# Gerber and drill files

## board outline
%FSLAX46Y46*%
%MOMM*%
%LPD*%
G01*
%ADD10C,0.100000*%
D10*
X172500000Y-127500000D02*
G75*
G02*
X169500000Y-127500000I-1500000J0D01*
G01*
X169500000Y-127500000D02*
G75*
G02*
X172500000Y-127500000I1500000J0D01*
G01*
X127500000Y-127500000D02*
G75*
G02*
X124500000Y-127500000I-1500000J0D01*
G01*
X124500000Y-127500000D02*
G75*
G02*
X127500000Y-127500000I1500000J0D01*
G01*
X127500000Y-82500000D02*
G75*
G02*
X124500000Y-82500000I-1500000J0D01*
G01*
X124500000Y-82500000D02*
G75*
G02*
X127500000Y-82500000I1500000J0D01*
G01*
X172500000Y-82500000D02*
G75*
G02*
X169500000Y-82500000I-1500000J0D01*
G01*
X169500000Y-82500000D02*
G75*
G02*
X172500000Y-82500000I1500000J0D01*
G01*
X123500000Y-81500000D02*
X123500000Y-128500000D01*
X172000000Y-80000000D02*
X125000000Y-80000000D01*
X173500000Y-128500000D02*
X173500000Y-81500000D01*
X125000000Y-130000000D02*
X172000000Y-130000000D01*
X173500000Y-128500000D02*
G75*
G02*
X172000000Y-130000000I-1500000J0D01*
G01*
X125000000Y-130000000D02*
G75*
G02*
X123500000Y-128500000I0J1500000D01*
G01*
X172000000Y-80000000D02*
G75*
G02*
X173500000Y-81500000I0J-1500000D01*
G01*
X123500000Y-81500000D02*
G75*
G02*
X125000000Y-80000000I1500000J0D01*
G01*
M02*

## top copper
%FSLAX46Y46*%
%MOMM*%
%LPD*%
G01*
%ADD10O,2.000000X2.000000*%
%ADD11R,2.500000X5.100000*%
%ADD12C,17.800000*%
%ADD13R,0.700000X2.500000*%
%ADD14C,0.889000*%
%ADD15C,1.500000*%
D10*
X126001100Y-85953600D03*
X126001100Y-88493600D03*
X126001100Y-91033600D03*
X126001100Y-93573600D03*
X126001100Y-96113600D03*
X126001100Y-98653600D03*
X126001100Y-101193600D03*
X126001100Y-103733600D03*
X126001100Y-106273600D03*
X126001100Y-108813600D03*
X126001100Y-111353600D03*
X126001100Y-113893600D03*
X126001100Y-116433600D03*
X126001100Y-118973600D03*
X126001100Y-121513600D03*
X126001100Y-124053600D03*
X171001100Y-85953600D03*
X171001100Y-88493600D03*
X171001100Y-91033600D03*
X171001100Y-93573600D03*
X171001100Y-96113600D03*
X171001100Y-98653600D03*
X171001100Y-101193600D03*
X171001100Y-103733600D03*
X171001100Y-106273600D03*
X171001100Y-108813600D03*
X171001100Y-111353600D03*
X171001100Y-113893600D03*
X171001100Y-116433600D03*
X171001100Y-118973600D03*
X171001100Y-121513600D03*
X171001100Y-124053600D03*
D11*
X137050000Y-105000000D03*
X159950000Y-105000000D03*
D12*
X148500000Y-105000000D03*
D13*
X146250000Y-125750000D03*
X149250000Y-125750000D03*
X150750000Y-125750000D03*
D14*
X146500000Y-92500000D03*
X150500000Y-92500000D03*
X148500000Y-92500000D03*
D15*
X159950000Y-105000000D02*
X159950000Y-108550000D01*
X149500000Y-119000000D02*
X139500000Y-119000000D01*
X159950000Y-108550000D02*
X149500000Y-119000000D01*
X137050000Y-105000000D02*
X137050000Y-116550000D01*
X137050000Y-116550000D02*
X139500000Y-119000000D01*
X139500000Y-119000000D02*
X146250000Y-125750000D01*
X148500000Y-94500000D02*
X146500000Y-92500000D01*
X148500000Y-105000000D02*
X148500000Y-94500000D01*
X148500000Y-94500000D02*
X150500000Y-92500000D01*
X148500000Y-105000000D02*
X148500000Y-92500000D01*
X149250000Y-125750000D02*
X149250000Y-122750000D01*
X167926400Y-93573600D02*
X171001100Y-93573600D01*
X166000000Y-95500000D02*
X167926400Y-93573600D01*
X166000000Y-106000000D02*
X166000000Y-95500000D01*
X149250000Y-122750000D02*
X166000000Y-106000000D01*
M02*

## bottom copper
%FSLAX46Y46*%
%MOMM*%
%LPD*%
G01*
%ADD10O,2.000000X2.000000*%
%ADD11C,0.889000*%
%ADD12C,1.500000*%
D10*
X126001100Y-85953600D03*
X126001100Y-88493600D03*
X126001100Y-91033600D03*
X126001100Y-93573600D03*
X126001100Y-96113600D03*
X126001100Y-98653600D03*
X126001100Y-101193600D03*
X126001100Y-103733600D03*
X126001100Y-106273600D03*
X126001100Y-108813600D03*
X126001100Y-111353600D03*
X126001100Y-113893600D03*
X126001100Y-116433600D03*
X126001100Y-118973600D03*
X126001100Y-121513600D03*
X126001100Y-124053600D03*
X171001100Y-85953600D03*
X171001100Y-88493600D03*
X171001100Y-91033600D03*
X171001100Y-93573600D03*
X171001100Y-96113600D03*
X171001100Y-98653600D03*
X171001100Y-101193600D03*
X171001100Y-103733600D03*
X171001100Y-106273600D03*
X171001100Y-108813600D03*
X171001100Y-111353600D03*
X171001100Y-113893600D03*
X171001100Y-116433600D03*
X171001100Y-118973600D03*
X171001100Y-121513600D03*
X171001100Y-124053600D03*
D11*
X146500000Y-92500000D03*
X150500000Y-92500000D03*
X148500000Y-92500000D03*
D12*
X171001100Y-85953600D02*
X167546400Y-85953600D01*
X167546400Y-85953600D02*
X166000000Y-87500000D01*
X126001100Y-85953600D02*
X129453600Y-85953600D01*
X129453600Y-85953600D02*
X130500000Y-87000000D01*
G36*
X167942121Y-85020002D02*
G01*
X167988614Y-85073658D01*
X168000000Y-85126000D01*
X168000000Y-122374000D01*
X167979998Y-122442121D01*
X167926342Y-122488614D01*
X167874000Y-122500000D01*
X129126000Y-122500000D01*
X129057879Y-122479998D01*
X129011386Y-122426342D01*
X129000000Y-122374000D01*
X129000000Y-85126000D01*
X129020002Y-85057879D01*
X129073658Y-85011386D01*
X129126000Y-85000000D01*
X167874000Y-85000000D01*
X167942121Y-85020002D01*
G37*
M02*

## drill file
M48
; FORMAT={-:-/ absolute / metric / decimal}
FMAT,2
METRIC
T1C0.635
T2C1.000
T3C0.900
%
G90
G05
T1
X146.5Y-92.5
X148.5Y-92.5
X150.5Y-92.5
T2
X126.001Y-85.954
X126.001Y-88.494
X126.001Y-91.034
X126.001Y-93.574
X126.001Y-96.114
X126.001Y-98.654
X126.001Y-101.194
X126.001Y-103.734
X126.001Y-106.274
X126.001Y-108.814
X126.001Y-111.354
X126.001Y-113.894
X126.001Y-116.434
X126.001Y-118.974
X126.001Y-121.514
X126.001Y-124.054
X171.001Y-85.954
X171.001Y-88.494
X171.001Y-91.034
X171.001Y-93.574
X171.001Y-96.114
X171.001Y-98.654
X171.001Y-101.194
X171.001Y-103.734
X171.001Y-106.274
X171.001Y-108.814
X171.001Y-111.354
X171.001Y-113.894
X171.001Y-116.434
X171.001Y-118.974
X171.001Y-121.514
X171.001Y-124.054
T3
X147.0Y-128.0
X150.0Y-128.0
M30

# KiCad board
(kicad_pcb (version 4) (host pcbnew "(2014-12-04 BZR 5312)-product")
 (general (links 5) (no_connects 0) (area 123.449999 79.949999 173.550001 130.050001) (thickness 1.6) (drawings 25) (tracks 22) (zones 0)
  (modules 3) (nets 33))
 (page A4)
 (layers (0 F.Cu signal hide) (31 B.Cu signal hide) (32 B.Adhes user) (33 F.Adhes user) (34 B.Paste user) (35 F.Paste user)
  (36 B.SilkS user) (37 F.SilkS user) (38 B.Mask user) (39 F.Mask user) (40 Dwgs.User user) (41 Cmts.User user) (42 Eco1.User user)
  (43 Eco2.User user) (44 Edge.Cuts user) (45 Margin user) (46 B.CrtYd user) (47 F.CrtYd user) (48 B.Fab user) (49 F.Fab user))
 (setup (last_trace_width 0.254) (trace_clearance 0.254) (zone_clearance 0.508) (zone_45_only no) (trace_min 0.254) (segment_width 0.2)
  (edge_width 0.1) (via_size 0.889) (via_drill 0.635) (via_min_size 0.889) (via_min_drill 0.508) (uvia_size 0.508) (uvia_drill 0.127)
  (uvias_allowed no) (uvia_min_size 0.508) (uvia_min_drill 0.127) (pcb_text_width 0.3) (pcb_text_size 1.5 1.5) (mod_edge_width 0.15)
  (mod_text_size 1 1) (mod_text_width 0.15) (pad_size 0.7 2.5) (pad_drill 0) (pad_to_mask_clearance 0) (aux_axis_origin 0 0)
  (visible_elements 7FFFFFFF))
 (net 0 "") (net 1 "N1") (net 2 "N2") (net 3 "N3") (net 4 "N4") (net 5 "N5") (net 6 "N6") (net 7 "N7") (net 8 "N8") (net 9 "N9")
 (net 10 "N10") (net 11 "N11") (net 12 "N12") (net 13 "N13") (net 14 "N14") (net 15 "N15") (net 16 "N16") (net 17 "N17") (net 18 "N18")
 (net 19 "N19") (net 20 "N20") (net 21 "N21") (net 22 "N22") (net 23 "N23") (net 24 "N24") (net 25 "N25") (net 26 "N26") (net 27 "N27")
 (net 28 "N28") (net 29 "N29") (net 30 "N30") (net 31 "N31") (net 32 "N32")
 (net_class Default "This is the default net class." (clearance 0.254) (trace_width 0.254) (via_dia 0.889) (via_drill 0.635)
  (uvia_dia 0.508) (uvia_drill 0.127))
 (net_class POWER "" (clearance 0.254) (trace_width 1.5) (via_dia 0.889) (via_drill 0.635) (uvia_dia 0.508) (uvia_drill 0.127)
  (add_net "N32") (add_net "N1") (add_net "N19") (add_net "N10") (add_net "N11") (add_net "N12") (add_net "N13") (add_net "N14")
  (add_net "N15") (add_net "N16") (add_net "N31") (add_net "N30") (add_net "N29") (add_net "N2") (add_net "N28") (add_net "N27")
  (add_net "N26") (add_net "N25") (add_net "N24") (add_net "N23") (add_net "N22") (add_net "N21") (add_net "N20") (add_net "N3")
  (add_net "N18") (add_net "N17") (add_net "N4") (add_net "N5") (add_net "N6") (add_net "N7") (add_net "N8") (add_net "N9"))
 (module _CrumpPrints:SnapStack (layer F.Cu) (at 148.5011 105.0036)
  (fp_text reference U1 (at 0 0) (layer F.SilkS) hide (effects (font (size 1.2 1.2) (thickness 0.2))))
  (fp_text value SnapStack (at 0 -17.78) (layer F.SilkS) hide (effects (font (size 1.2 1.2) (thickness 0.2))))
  (pad 1 thru_hole oval (at -22.5 -19.05) (size 2 2) (drill 1) (layers *.Cu *.Mask F.SilkS) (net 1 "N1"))
  (pad 2 thru_hole oval (at -22.5 -16.51) (size 2 2) (drill 1) (layers *.Cu *.Mask F.SilkS) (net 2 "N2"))
  (pad 3 thru_hole oval (at -22.5 -13.97) (size 2 2) (drill 1) (layers *.Cu *.Mask F.SilkS) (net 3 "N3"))
  (pad 4 thru_hole oval (at -22.5 -11.43) (size 2 2) (drill 1) (layers *.Cu *.Mask F.SilkS) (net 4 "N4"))
  (pad 5 thru_hole oval (at -22.5 -8.89) (size 2 2) (drill 1) (layers *.Cu *.Mask F.SilkS) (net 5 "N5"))
  (pad 6 thru_hole oval (at -22.5 -6.35) (size 2 2) (drill 1) (layers *.Cu *.Mask F.SilkS) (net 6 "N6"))
  (pad 7 thru_hole oval (at -22.5 -3.81) (size 2 2) (drill 1) (layers *.Cu *.Mask F.SilkS) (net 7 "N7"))
  (pad 8 thru_hole oval (at -22.5 -1.27) (size 2 2) (drill 1) (layers *.Cu *.Mask F.SilkS) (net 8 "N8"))
  (pad 9 thru_hole oval (at -22.5 1.27) (size 2 2) (drill 1) (layers *.Cu *.Mask F.SilkS) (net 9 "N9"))
  (pad 10 thru_hole oval (at -22.5 3.81) (size 2 2) (drill 1) (layers *.Cu *.Mask F.SilkS) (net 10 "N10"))
  (pad 11 thru_hole oval (at -22.5 6.35) (size 2 2) (drill 1) (layers *.Cu *.Mask F.SilkS) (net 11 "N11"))
  (pad 12 thru_hole oval (at -22.5 8.89) (size 2 2) (drill 1) (layers *.Cu *.Mask F.SilkS) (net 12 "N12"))
  (pad 13 thru_hole oval (at -22.5 11.43) (size 2 2) (drill 1) (layers *.Cu *.Mask F.SilkS) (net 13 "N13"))
  (pad 14 thru_hole oval (at -22.5 13.97) (size 2 2) (drill 1) (layers *.Cu *.Mask F.SilkS) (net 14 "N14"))
  (pad 15 thru_hole oval (at -22.5 16.51) (size 2 2) (drill 1) (layers *.Cu *.Mask F.SilkS) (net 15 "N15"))
  (pad 16 thru_hole oval (at -22.5 19.05) (size 2 2) (drill 1) (layers *.Cu *.Mask F.SilkS) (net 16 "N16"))
  (pad 32 thru_hole oval (at 22.5 -19.05) (size 2 2) (drill 1) (layers *.Cu *.Mask F.SilkS) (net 1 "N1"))
  (pad 31 thru_hole oval (at 22.5 -16.51) (size 2 2) (drill 1) (layers *.Cu *.Mask F.SilkS) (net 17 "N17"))
  (pad 30 thru_hole oval (at 22.5 -13.97) (size 2 2) (drill 1) (layers *.Cu *.Mask F.SilkS) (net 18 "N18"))
  (pad 29 thru_hole oval (at 22.5 -11.43) (size 2 2) (drill 1) (layers *.Cu *.Mask F.SilkS) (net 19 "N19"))
  (pad 28 thru_hole oval (at 22.5 -8.89) (size 2 2) (drill 1) (layers *.Cu *.Mask F.SilkS) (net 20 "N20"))
  (pad 27 thru_hole oval (at 22.5 -6.35) (size 2 2) (drill 1) (layers *.Cu *.Mask F.SilkS) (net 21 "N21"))
  (pad 26 thru_hole oval (at 22.5 -3.81) (size 2 2) (drill 1) (layers *.Cu *.Mask F.SilkS) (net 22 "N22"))
  (pad 25 thru_hole oval (at 22.5 -1.27) (size 2 2) (drill 1) (layers *.Cu *.Mask F.SilkS) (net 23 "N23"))
  (pad 24 thru_hole oval (at 22.5 1.27) (size 2 2) (drill 1) (layers *.Cu *.Mask F.SilkS) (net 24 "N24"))
  (pad 23 thru_hole oval (at 22.5 3.81) (size 2 2) (drill 1) (layers *.Cu *.Mask F.SilkS) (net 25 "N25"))
  (pad 22 thru_hole oval (at 22.5 6.35) (size 2 2) (drill 1) (layers *.Cu *.Mask F.SilkS) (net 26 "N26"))
  (pad 21 thru_hole oval (at 22.5 8.89) (size 2 2) (drill 1) (layers *.Cu *.Mask F.SilkS) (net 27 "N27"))
  (pad 20 thru_hole oval (at 22.5 11.43) (size 2 2) (drill 1) (layers *.Cu *.Mask F.SilkS) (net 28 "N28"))
  (pad 19 thru_hole oval (at 22.5 13.97) (size 2 2) (drill 1) (layers *.Cu *.Mask F.SilkS) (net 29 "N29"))
  (pad 18 thru_hole oval (at 22.5 16.51) (size 2 2) (drill 1) (layers *.Cu *.Mask F.SilkS) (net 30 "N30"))
  (pad 17 thru_hole oval (at 22.5 19.05) (size 2 2) (drill 1) (layers *.Cu *.Mask F.SilkS) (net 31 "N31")))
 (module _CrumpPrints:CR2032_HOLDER (layer F.Cu) (at 148.5 105)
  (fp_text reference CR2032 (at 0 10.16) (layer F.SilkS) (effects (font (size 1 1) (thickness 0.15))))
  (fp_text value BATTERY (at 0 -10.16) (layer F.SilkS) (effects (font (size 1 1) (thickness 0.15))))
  (pad 1 smd rect (at -11.45 0) (size 2.5 5.1) (layers F.Cu F.Paste F.Mask) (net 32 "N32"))
  (pad 1 smd rect (at 11.45 0) (size 2.5 5.1) (layers F.Cu F.Paste F.Mask) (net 32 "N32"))
  (pad 2 smd circle (at 0 0) (size 17.8 17.8) (layers F.Cu F.Paste F.Mask) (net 1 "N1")))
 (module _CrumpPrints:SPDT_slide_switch (layer F.Cu) (at 148.5 128)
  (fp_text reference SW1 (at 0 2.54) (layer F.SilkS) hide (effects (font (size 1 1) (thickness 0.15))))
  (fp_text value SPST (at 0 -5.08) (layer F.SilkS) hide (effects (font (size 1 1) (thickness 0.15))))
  (pad "" np_thru_hole circle (at 1.5 0) (size 0.9 0.9) (drill 0.9) (layers *.Cu *.Mask F.SilkS))
  (pad "" np_thru_hole circle (at -1.5 0) (size 0.9 0.9) (drill 0.9) (layers *.Cu *.Mask F.SilkS))
  (pad 1 smd rect (at -2.25 -2.25) (size 0.7 2.5) (layers F.Cu F.Paste F.Mask) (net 32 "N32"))
  (pad 2 smd rect (at 0.75 -2.25) (size 0.7 2.5) (layers F.Cu F.Paste F.Mask) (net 19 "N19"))
  (pad 3 smd rect (at 2.25 -2.25) (size 0.7 2.5) (layers F.Cu F.Paste F.Mask)))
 (gr_circle (center 171 127.5) (end 171 129) (layer Edge.Cuts) (width 0.1))
 (gr_circle (center 126 127.5) (end 126 126) (layer Edge.Cuts) (width 0.1))
 (gr_circle (center 126 82.5) (end 126 81) (layer Edge.Cuts) (width 0.1))
 (gr_circle (center 171 82.5) (end 169.5 82.5) (layer Edge.Cuts) (width 0.1))
 (gr_line (start 123.5 81.5) (end 123.5 128.5) (angle 90) (layer Edge.Cuts) (width 0.1))
 (gr_line (start 172 80) (end 125 80) (angle 90) (layer Edge.Cuts) (width 0.1))
 (gr_line (start 173.5 128.5) (end 173.5 81.5) (angle 90) (layer Edge.Cuts) (width 0.1))
 (gr_line (start 125 130) (end 172 130) (angle 90) (layer Edge.Cuts) (width 0.1))
 (gr_arc (start 172 128.5) (end 173.5 128.5) (angle 90) (layer Edge.Cuts) (width 0.1))
 (gr_arc (start 125 128.5) (end 125 130) (angle 90) (layer Edge.Cuts) (width 0.1))
 (gr_arc (start 172 81.5) (end 172 80) (angle 90) (layer Edge.Cuts) (width 0.1))
 (gr_arc (start 125 81.5) (end 123.5 81.5) (angle 90) (layer Edge.Cuts) (width 0.1))
 (segment (start 159.95 105) (end 159.95 108.55) (width 1.5) (layer F.Cu) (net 32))
 (segment (start 149.5 119) (end 139.5 119) (width 1.5) (layer F.Cu) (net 32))
 (segment (start 159.95 108.55) (end 149.5 119) (width 1.5) (layer F.Cu) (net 32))
 (segment (start 137.05 105) (end 137.05 116.55) (width 1.5) (layer F.Cu) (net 32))
 (segment (start 137.05 116.55) (end 139.5 119) (width 1.5) (layer F.Cu) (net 32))
 (segment (start 139.5 119) (end 146.25 125.75) (width 1.5) (layer F.Cu) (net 32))
 (segment (start 171.0011 85.9536) (end 167.5464 85.9536) (width 1.5) (layer B.Cu) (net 1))
 (segment (start 167.5464 85.9536) (end 166 87.5) (width 1.5) (layer B.Cu) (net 1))
 (segment (start 126.0011 85.9536) (end 129.4536 85.9536) (width 1.5) (layer B.Cu) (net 1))
 (segment (start 129.4536 85.9536) (end 130.5 87) (width 1.5) (layer B.Cu) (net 1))
 (segment (start 148.5 94.5) (end 146.5 92.5) (width 1.5) (layer F.Cu) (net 1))
 (via (at 146.5 92.5) (size 0.889) (layers F.Cu B.Cu) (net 1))
 (segment (start 148.5 105) (end 148.5 94.5) (width 1.5) (layer F.Cu) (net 1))
 (via (at 150.5 92.5) (size 0.889) (layers F.Cu B.Cu) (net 1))
 (segment (start 148.5 94.5) (end 150.5 92.5) (width 1.5) (layer F.Cu) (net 1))
 (segment (start 148.5 105) (end 148.5 92.5) (width 1.5) (layer F.Cu) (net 1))
 (via (at 148.5 92.5) (size 0.889) (layers F.Cu B.Cu) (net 1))
 (segment (start 149.25 125.75) (end 149.25 122.75) (width 1.5) (layer F.Cu) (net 19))
 (segment (start 167.9264 93.5736) (end 171.0011 93.5736) (width 1.5) (layer F.Cu) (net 19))
 (segment (start 166 95.5) (end 167.9264 93.5736) (width 1.5) (layer F.Cu) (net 19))
 (segment (start 166 106) (end 166 95.5) (width 1.5) (layer F.Cu) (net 19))
 (segment (start 149.25 122.75) (end 166 106) (width 1.5) (layer F.Cu) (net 19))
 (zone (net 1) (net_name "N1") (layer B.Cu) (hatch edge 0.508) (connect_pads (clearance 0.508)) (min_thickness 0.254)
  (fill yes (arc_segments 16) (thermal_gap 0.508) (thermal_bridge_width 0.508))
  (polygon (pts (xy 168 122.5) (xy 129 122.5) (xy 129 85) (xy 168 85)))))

